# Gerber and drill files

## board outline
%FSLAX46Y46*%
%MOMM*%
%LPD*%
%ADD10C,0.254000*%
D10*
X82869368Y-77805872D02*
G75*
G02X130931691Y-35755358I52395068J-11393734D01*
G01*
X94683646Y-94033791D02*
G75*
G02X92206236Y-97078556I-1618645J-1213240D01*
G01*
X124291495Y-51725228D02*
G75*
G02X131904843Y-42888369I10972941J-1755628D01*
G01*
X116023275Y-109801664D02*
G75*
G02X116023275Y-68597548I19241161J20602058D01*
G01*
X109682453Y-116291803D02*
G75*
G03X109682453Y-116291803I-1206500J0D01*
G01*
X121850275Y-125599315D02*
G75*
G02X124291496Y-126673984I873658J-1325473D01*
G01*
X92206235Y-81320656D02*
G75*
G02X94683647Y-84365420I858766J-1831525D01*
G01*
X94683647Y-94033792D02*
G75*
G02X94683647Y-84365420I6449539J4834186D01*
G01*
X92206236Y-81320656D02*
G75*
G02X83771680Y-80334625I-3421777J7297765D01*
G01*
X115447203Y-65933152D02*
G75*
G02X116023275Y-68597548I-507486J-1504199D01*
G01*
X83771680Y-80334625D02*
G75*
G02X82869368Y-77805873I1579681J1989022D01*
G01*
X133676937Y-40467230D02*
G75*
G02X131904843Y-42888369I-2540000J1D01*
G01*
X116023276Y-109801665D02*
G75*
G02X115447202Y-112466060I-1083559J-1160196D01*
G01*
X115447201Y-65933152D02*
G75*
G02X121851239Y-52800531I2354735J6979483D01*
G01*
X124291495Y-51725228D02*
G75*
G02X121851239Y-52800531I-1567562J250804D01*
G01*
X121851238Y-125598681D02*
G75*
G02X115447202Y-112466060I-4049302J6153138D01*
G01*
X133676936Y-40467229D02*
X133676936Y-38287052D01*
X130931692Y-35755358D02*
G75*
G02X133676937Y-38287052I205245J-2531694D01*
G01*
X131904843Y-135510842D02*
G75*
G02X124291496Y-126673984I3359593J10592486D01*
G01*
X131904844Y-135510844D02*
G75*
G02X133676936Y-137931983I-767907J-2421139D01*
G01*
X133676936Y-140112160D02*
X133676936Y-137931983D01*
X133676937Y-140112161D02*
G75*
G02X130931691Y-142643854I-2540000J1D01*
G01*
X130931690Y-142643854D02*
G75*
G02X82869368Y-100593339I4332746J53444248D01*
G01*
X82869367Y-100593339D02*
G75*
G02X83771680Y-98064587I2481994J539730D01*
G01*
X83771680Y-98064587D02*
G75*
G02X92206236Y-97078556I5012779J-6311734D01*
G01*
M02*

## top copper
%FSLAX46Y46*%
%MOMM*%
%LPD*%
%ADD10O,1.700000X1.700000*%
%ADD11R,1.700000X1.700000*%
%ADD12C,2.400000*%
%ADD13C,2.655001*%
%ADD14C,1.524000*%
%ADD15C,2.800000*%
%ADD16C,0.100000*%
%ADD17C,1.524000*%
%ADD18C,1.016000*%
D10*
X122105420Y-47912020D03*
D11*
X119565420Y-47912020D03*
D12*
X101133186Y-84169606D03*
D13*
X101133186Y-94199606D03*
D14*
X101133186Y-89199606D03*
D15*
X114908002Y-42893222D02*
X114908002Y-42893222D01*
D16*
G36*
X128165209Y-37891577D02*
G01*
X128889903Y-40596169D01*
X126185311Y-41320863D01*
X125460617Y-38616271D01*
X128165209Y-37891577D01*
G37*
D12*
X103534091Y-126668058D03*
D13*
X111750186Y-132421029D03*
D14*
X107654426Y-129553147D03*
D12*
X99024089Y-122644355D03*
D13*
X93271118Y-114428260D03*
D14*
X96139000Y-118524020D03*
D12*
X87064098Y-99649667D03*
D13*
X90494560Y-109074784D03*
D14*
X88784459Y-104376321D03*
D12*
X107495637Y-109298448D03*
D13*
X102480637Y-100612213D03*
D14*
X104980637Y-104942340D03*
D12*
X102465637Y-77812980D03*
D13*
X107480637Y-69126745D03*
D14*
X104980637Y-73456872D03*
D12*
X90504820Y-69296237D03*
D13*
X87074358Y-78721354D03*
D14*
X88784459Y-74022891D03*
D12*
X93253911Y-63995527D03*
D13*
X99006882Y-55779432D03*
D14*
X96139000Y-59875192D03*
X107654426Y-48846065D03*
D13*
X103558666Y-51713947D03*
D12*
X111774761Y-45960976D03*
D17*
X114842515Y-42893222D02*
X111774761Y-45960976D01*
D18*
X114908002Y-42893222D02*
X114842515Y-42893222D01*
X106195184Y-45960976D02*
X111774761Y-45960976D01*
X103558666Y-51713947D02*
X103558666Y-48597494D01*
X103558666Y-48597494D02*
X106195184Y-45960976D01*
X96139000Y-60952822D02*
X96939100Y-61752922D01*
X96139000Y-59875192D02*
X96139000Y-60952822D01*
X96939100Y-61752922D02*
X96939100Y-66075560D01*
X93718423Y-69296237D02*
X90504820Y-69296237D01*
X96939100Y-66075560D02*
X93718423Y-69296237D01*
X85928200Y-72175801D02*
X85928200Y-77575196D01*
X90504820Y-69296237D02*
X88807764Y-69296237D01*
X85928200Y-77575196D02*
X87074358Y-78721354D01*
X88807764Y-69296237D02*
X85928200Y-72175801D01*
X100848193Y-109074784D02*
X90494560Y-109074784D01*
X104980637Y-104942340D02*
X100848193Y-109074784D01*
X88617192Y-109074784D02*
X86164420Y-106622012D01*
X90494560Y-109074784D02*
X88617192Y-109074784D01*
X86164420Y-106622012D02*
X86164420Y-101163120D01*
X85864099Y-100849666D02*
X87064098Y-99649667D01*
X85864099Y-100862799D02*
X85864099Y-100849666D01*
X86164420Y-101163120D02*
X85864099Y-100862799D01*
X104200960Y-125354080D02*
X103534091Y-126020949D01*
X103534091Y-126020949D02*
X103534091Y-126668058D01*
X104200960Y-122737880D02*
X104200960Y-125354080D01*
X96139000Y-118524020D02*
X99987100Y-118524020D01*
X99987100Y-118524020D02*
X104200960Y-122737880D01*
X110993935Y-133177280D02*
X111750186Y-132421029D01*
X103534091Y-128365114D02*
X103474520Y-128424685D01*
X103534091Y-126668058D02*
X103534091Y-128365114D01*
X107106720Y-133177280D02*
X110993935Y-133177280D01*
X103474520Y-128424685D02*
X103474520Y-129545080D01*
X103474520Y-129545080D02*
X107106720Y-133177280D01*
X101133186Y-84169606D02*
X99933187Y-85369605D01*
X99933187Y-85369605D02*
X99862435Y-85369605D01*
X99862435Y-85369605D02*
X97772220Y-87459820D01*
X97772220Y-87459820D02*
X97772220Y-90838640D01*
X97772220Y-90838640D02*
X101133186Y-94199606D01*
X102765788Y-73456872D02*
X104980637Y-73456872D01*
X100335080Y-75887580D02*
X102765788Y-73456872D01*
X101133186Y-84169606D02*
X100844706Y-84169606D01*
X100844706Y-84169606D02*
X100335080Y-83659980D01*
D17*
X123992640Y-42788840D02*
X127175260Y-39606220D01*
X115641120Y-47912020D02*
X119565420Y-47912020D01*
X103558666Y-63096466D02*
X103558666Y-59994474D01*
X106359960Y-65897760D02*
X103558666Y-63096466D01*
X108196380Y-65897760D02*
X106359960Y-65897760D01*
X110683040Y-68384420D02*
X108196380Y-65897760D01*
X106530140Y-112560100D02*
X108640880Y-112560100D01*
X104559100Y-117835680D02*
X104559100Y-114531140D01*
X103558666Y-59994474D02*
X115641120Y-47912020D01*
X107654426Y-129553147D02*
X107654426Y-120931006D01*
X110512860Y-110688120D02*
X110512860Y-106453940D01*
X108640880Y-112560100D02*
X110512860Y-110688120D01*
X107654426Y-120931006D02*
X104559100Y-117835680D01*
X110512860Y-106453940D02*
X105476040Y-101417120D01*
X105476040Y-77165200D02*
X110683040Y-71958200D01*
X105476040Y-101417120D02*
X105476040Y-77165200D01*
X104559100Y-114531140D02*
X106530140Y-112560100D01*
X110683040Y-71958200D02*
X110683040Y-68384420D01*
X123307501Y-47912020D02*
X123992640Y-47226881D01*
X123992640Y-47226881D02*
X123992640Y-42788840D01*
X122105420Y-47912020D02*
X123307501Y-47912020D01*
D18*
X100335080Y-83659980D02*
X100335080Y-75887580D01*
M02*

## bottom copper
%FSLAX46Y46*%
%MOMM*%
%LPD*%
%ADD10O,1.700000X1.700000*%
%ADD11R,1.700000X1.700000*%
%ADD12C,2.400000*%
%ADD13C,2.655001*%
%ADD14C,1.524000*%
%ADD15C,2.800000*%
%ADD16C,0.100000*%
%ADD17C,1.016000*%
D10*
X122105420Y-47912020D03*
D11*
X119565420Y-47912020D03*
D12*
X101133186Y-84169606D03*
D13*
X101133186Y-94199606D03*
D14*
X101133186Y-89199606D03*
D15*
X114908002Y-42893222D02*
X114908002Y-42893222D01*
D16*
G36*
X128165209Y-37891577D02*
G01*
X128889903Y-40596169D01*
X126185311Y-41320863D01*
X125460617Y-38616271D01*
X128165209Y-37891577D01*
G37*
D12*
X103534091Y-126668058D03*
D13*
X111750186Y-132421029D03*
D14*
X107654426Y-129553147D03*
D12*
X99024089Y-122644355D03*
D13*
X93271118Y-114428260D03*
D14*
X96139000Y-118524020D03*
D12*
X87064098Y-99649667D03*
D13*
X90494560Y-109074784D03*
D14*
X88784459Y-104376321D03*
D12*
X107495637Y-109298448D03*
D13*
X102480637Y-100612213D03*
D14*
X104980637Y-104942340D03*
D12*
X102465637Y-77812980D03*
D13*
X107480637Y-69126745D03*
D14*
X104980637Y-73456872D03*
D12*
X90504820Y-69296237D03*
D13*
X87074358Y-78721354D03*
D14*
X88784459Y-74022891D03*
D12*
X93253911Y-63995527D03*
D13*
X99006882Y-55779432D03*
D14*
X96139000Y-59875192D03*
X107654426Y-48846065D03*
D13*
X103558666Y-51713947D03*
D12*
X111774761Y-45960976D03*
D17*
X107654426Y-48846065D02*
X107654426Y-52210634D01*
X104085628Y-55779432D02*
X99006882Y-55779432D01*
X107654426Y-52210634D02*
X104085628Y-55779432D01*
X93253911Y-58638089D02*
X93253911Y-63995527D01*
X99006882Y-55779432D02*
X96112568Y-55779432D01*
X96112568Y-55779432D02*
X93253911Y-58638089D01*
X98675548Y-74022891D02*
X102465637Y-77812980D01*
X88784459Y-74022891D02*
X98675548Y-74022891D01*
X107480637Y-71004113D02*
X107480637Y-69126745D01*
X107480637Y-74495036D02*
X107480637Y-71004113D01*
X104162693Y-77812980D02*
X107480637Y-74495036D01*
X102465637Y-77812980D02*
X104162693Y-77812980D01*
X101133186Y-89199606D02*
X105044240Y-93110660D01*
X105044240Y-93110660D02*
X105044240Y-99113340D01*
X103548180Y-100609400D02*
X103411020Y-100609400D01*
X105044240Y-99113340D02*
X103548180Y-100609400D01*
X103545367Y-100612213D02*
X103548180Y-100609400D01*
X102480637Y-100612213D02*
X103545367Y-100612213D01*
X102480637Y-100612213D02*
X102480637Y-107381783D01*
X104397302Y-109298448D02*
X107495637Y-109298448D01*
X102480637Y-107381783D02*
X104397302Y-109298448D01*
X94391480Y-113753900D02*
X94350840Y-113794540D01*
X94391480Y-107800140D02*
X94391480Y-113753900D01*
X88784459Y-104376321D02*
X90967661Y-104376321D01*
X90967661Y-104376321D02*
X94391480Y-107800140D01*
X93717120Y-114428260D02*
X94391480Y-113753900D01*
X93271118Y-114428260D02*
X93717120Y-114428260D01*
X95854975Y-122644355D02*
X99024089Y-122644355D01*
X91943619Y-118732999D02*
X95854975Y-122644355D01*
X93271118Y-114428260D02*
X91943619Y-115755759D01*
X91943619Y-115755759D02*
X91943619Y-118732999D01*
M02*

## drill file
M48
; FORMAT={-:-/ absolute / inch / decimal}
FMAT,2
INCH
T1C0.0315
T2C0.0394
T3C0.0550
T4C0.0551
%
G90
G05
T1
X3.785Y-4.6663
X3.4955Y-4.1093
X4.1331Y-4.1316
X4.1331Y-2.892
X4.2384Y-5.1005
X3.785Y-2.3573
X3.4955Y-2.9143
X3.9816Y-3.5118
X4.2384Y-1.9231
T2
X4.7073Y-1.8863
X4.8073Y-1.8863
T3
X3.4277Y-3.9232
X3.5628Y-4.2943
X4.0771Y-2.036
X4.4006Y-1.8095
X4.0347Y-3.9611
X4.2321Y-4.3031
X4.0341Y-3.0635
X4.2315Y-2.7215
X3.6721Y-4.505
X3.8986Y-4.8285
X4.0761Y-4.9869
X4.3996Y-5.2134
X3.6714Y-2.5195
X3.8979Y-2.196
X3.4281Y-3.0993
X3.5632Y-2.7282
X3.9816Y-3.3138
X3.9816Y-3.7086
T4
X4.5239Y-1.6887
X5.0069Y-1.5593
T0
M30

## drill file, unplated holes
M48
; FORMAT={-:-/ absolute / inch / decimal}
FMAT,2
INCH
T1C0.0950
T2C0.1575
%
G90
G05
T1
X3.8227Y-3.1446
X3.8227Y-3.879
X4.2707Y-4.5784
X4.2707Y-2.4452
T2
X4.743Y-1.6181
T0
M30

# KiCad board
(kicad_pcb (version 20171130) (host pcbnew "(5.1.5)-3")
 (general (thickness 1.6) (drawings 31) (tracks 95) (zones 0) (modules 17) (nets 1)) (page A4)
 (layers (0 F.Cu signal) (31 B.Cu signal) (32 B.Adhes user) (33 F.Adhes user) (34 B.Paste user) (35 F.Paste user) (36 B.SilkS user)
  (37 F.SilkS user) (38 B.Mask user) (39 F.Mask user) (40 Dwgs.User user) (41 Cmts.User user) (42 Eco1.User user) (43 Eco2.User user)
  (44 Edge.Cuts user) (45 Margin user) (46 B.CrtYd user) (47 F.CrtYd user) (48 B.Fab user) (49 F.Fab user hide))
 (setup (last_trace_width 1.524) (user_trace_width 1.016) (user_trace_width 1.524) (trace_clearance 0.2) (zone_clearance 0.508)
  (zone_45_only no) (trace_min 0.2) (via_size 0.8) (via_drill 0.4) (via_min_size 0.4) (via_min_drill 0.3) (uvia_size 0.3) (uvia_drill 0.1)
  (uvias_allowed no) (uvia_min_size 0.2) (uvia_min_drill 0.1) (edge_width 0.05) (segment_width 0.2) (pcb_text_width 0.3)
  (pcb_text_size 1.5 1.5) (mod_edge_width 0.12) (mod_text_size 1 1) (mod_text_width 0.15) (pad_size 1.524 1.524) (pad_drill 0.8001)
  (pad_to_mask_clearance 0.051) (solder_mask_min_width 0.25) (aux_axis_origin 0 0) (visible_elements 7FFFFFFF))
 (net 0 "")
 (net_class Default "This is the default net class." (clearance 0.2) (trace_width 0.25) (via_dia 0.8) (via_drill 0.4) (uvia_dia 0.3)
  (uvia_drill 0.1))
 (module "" (layer F.Cu) (at 121.2342 50.3174)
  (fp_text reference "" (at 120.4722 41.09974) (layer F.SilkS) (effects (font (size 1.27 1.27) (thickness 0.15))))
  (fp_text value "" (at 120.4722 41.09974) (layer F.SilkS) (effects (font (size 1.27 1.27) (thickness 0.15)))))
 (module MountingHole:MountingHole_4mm (layer F.Cu) (at 120.4722 41.09974)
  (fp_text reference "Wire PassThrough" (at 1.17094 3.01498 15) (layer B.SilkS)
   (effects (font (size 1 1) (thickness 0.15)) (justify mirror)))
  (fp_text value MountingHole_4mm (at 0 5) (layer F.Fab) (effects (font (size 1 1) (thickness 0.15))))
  (pad "" np_thru_hole circle (at 0 0) (size 4 4) (drill 4) (layers *.Cu *.Mask)))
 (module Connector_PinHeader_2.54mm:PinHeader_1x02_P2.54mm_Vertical (layer F.Cu) (at 119.56542 47.91202 90)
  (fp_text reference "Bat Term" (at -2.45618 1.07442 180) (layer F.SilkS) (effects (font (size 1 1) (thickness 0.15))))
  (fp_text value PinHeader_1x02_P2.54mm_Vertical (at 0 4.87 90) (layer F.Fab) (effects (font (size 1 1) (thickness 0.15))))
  (pad 2 thru_hole oval (at 0 2.54 90) (size 1.7 1.7) (drill 1) (layers *.Cu *.Mask))
  (pad 1 thru_hole rect (at 0 0 90) (size 1.7 1.7) (drill 1) (layers *.Cu *.Mask)))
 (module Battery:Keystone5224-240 (layer F.Cu) (at 101.133186 89.199606)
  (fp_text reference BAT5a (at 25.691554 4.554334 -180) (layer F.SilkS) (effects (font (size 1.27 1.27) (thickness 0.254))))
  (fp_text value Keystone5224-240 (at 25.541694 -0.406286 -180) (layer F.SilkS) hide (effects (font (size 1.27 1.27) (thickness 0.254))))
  (pad 2 thru_hole circle (at 0 -5.03) (size 2.4 2.4) (drill 1.397) (layers *.Cu *.Mask))
  (pad 1 thru_hole circle (at 0 5) (size 2.655001 2.655001) (drill 1.397) (layers *.Cu *.Mask))
  (pad 3 thru_hole circle (at 0 0) (size 1.524 1.524) (drill 0.8001) (layers *.Cu *.Mask)))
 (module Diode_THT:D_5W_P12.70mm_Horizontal (layer F.Cu) (at 127.17526 39.60622 195)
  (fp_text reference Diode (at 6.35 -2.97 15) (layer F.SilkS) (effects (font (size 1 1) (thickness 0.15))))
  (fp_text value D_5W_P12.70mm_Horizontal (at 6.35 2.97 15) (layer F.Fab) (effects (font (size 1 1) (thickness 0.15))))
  (pad 2 thru_hole oval (at 12.7 0 195) (size 2.8 2.8) (drill 1.4) (layers *.Cu *.Mask))
  (pad 1 thru_hole rect (at 0 0 195) (size 2.8 2.8) (drill 1.4) (layers *.Cu *.Mask)))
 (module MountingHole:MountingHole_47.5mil (layer F.Cu) (at 108.475953 116.291803)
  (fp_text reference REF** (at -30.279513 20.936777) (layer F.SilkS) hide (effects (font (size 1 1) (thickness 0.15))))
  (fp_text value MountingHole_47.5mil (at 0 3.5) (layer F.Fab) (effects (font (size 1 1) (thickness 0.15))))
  (pad "" np_thru_hole circle (at 0 0) (size 2.413 2.413) (drill 2.413) (layers *.Cu *.Mask)))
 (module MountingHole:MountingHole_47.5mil (layer F.Cu) (at 97.096838 98.527587)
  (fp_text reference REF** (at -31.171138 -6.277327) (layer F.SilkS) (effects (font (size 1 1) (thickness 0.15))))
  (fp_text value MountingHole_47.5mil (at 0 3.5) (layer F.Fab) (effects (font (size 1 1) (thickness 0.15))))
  (pad "" np_thru_hole circle (at 0 0) (size 2.413 2.413) (drill 2.413) (layers *.Cu *.Mask)))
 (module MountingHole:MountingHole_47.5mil (layer F.Cu) (at 97.096838 79.871625)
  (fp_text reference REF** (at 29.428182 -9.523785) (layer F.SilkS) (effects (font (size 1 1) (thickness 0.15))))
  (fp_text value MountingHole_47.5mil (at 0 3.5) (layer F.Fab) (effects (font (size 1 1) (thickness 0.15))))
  (pad "" np_thru_hole circle (at 0 0) (size 2.413 2.413) (drill 2.413) (layers *.Cu *.Mask)))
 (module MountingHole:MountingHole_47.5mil (layer F.Cu) (at 108.475953 62.107409)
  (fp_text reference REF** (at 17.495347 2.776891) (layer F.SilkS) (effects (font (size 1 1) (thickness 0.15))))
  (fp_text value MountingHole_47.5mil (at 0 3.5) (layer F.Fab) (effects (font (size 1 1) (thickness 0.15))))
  (pad "" np_thru_hole circle (at 0 0) (size 2.413 2.413) (drill 2.413) (layers *.Cu *.Mask)))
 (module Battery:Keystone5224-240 (layer F.Cu) (at 107.654426 129.553147 55)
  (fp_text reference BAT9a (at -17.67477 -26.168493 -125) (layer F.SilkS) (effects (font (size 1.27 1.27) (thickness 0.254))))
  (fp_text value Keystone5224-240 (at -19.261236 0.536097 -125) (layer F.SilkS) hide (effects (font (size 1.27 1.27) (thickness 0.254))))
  (pad 2 thru_hole circle (at 0 -5.03 55) (size 2.4 2.4) (drill 1.397) (layers *.Cu *.Mask))
  (pad 1 thru_hole circle (at 0 5 55) (size 2.655001 2.655001) (drill 1.397) (layers *.Cu *.Mask))
  (pad 3 thru_hole circle (at 0 0 55) (size 1.524 1.524) (drill 0.8001) (layers *.Cu *.Mask)))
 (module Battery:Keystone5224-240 (layer B.Cu) (at 96.139 118.52402 35)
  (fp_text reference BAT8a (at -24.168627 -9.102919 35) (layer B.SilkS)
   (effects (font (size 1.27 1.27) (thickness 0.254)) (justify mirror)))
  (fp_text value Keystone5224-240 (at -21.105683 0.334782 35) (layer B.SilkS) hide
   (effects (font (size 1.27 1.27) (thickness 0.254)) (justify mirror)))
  (pad 2 thru_hole circle (at 0 5.03 35) (size 2.4 2.4) (drill 1.397) (layers *.Cu *.Mask))
  (pad 1 thru_hole circle (at 0 -5 35) (size 2.655001 2.655001) (drill 1.397) (layers *.Cu *.Mask))
  (pad 3 thru_hole circle (at 0 0 35) (size 1.524 1.524) (drill 0.8001) (layers *.Cu *.Mask)))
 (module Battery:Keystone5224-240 (layer F.Cu) (at 88.784459 104.376321 20)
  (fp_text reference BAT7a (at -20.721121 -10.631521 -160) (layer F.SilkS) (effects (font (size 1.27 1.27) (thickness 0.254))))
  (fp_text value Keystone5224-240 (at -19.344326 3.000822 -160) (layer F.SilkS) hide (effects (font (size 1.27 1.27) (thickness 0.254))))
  (pad 2 thru_hole circle (at 0 -5.03 20) (size 2.4 2.4) (drill 1.397) (layers *.Cu *.Mask))
  (pad 1 thru_hole circle (at 0 5 20) (size 2.655001 2.655001) (drill 1.397) (layers *.Cu *.Mask))
  (pad 3 thru_hole circle (at 0 0 20) (size 1.524 1.524) (drill 0.8001) (layers *.Cu *.Mask)))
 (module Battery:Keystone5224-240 (layer B.Cu) (at 104.980637 104.94234 30)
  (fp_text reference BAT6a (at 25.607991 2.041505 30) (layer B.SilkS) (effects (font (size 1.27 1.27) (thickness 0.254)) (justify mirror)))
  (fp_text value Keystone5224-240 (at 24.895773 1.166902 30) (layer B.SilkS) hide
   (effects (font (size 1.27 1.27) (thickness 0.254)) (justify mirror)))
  (pad 2 thru_hole circle (at 0 5.03 30) (size 2.4 2.4) (drill 1.397) (layers *.Cu *.Mask))
  (pad 1 thru_hole circle (at 0 -5 30) (size 2.655001 2.655001) (drill 1.397) (layers *.Cu *.Mask))
  (pad 3 thru_hole circle (at 0 0 30) (size 1.524 1.524) (drill 0.8001) (layers *.Cu *.Mask)))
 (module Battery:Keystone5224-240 (layer B.Cu) (at 104.980637 73.456872 330)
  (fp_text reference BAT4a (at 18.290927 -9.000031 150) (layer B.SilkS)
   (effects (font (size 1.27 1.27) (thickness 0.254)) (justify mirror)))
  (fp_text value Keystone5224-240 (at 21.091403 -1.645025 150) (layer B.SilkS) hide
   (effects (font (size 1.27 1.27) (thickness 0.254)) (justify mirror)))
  (pad 2 thru_hole circle (at 0 5.03 330) (size 2.4 2.4) (drill 1.397) (layers *.Cu *.Mask))
  (pad 1 thru_hole circle (at 0 -5 330) (size 2.655001 2.655001) (drill 1.397) (layers *.Cu *.Mask))
  (pad 3 thru_hole circle (at 0 0 330) (size 1.524 1.524) (drill 0.8001) (layers *.Cu *.Mask)))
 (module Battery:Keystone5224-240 (layer F.Cu) (at 88.784459 74.022891 340)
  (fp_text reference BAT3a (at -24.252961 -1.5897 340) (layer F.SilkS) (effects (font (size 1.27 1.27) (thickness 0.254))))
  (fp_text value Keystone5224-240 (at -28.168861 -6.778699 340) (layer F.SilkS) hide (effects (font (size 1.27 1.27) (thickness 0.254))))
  (pad 2 thru_hole circle (at 0 -5.03 340) (size 2.4 2.4) (drill 1.397) (layers *.Cu *.Mask))
  (pad 1 thru_hole circle (at 0 5 340) (size 2.655001 2.655001) (drill 1.397) (layers *.Cu *.Mask))
  (pad 3 thru_hole circle (at 0 0 340) (size 1.524 1.524) (drill 0.8001) (layers *.Cu *.Mask)))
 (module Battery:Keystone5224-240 (layer B.Cu) (at 96.139 59.875192 325)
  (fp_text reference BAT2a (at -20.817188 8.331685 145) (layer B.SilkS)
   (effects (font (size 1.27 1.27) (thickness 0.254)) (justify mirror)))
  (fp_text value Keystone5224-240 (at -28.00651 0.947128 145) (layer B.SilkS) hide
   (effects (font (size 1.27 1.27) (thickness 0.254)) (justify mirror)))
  (pad 2 thru_hole circle (at 0 5.03 325) (size 2.4 2.4) (drill 1.397) (layers *.Cu *.Mask))
  (pad 1 thru_hole circle (at 0 -5 325) (size 2.655001 2.655001) (drill 1.397) (layers *.Cu *.Mask))
  (pad 3 thru_hole circle (at 0 0 325) (size 1.524 1.524) (drill 0.8001) (layers *.Cu *.Mask)))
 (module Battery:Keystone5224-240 (layer F.Cu) (at 107.654426 48.846065 305)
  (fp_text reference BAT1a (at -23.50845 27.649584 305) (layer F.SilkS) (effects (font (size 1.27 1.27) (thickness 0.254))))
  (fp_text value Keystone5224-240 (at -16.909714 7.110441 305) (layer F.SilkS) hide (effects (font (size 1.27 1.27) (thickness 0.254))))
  (pad 3 thru_hole circle (at 0 0 305) (size 1.524 1.524) (drill 0.8001) (layers *.Cu *.Mask))
  (pad 1 thru_hole circle (at 0 5 305) (size 2.655001 2.655001) (drill 1.397) (layers *.Cu *.Mask))
  (pad 2 thru_hole circle (at 0 -5.03 305) (size 2.4 2.4) (drill 1.397) (layers *.Cu *.Mask)))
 (gr_arc (start 135.264436 89.199606) (end 130.931691 35.755358) (angle -73.09671633) (layer Edge.Cuts) (width 0.254))
 (gr_arc (start 93.065001 95.247031) (end 92.206236 97.078556) (angle -151.9739674) (layer Edge.Cuts) (width 0.254))
 (gr_arc (start 135.264436 53.480856) (end 131.904843 42.888369) (angle -63.31259973) (layer Edge.Cuts) (width 0.254))
 (gr_arc (start 135.264436 89.199606) (end 116.023275 68.597548) (angle -93.91250265) (layer Edge.Cuts) (width 0.254))
 (gr_circle (center 108.475953 116.291803) (end 109.682453 116.291803) (layer Edge.Cuts) (width 0.254))
 (gr_arc (start 122.723933 126.924788) (end 124.291496 126.673984) (angle -114.3) (layer Edge.Cuts) (width 0.254))
 (gr_arc (start 93.065001 83.152181) (end 94.683647 84.36542) (angle -151.9739674) (layer Edge.Cuts) (width 0.254))
 (gr_arc (start 101.133186 89.199606) (end 94.683647 84.36542) (angle -73.70603612) (layer Edge.Cuts) (width 0.254))
 (gr_arc (start 88.784459 74.022891) (end 83.77168 80.334625) (angle -63.5775508) (layer Edge.Cuts) (width 0.254))
 (gr_arc (start 114.939717 67.437351) (end 116.023275 68.597548) (angle -118.3129136) (layer Edge.Cuts) (width 0.254))
 (gr_arc (start 85.351361 78.345603) (end 82.869368 77.805873) (angle -63.8118281) (layer Edge.Cuts) (width 0.254))
 (gr_arc (start 131.136937 40.467229) (end 131.904843 42.888369) (angle -72.40266339) (layer Edge.Cuts) (width 0.254))
 (gr_arc (start 114.939717 110.961861) (end 115.447202 112.46606) (angle -118.3129136) (layer Edge.Cuts) (width 0.254))
 (gr_arc (start 117.801936 58.953669) (end 121.851239 52.800531) (angle -194.7050695) (layer Edge.Cuts) (width 0.254))
 (gr_arc (start 122.723933 51.474424) (end 121.851239 52.800531) (angle -114.2583435) (layer Edge.Cuts) (width 0.254))
 (gr_arc (start 117.801936 119.445543) (end 115.447202 112.46606) (angle -194.7050695) (layer Edge.Cuts) (width 0.254))
 (gr_line (start 133.676936 40.467229) (end 133.676936 38.287052) (layer Edge.Cuts) (width 0.254))
 (gr_arc (start 131.136937 38.287052) (end 133.676937 38.287052) (angle -94.63485415) (layer Edge.Cuts) (width 0.254))
 (gr_arc (start 135.264436 124.918356) (end 124.291496 126.673984) (angle -63.31259973) (layer Edge.Cuts) (width 0.254))
 (gr_arc (start 131.136937 137.931983) (end 133.676936 137.931983) (angle -72.40266339) (layer Edge.Cuts) (width 0.254))
 (gr_line (start 133.676936 140.11216) (end 133.676936 137.931983) (layer Edge.Cuts) (width 0.254))
 (gr_arc (start 131.136937 140.11216) (end 130.931691 142.643854) (angle -94.63485415) (layer Edge.Cuts) (width 0.254))
 (gr_arc (start 135.264436 89.199606) (end 82.869368 100.593339) (angle -73.09671633) (layer Edge.Cuts) (width 0.254))
 (gr_arc (start 85.351361 100.053609) (end 83.77168 98.064587) (angle -63.8118281) (layer Edge.Cuts) (width 0.254))
 (gr_arc (start 88.784459 104.376321) (end 92.206236 97.078556) (angle -63.5775508) (layer Edge.Cuts) (width 0.254))
 (segment (start 114.842515 42.893222) (end 111.774761 45.960976) (width 1.524) (layer F.Cu) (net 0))
 (segment (start 114.908002 42.893222) (end 114.842515 42.893222) (width 1.016) (layer F.Cu) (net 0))
 (segment (start 106.195184 45.960976) (end 111.774761 45.960976) (width 1.016) (layer F.Cu) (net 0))
 (segment (start 103.558666 51.713947) (end 103.558666 48.597494) (width 1.016) (layer F.Cu) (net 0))
 (segment (start 103.558666 48.597494) (end 106.195184 45.960976) (width 1.016) (layer F.Cu) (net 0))
 (segment (start 107.654426 48.846065) (end 107.654426 52.210634) (width 1.016) (layer B.Cu) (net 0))
 (segment (start 104.085628 55.779432) (end 99.006882 55.779432) (width 1.016) (layer B.Cu) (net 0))
 (segment (start 107.654426 52.210634) (end 104.085628 55.779432) (width 1.016) (layer B.Cu) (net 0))
 (segment (start 93.253911 58.638089) (end 93.253911 63.995527) (width 1.016) (layer B.Cu) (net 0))
 (segment (start 99.006882 55.779432) (end 96.112568 55.779432) (width 1.016) (layer B.Cu) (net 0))
 (segment (start 96.112568 55.779432) (end 93.253911 58.638089) (width 1.016) (layer B.Cu) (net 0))
 (segment (start 96.139 60.952822) (end 96.9391 61.752922) (width 1.016) (layer F.Cu) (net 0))
 (segment (start 96.139 59.875192) (end 96.139 60.952822) (width 1.016) (layer F.Cu) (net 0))
 (segment (start 96.9391 61.752922) (end 96.9391 66.07556) (width 1.016) (layer F.Cu) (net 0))
 (segment (start 93.718423 69.296237) (end 90.50482 69.296237) (width 1.016) (layer F.Cu) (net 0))
 (segment (start 96.9391 66.07556) (end 93.718423 69.296237) (width 1.016) (layer F.Cu) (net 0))
 (segment (start 85.9282 72.175801) (end 85.9282 77.575196) (width 1.016) (layer F.Cu) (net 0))
 (segment (start 90.50482 69.296237) (end 88.807764 69.296237) (width 1.016) (layer F.Cu) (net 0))
 (segment (start 85.9282 77.575196) (end 87.074358 78.721354) (width 1.016) (layer F.Cu) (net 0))
 (segment (start 88.807764 69.296237) (end 85.9282 72.175801) (width 1.016) (layer F.Cu) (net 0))
 (segment (start 100.848193 109.074784) (end 90.49456 109.074784) (width 1.016) (layer F.Cu) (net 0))
 (segment (start 104.980637 104.94234) (end 100.848193 109.074784) (width 1.016) (layer F.Cu) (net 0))
 (segment (start 88.617192 109.074784) (end 86.16442 106.622012) (width 1.016) (layer F.Cu) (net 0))
 (segment (start 90.49456 109.074784) (end 88.617192 109.074784) (width 1.016) (layer F.Cu) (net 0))
 (segment (start 86.16442 106.622012) (end 86.16442 101.16312) (width 1.016) (layer F.Cu) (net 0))
 (segment (start 85.864099 100.849666) (end 87.064098 99.649667) (width 1.016) (layer F.Cu) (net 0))
 (segment (start 85.864099 100.862799) (end 85.864099 100.849666) (width 1.016) (layer F.Cu) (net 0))
 (segment (start 86.16442 101.16312) (end 85.864099 100.862799) (width 1.016) (layer F.Cu) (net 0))
 (segment (start 104.20096 125.35408) (end 103.534091 126.020949) (width 1.016) (layer F.Cu) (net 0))
 (segment (start 103.534091 126.020949) (end 103.534091 126.668058) (width 1.016) (layer F.Cu) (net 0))
 (segment (start 104.20096 122.73788) (end 104.20096 125.35408) (width 1.016) (layer F.Cu) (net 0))
 (segment (start 96.139 118.52402) (end 99.9871 118.52402) (width 1.016) (layer F.Cu) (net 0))
 (segment (start 99.9871 118.52402) (end 104.20096 122.73788) (width 1.016) (layer F.Cu) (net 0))
 (segment (start 110.993935 133.17728) (end 111.750186 132.421029) (width 1.016) (layer F.Cu) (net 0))
 (segment (start 103.534091 128.365114) (end 103.47452 128.424685) (width 1.016) (layer F.Cu) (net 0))
 (segment (start 103.534091 126.668058) (end 103.534091 128.365114) (width 1.016) (layer F.Cu) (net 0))
 (segment (start 107.10672 133.17728) (end 110.993935 133.17728) (width 1.016) (layer F.Cu) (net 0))
 (segment (start 103.47452 128.424685) (end 103.47452 129.54508) (width 1.016) (layer F.Cu) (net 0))
 (segment (start 103.47452 129.54508) (end 107.10672 133.17728) (width 1.016) (layer F.Cu) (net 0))
 (segment (start 98.675548 74.022891) (end 102.465637 77.81298) (width 1.016) (layer B.Cu) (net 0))
 (segment (start 88.784459 74.022891) (end 98.675548 74.022891) (width 1.016) (layer B.Cu) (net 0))
 (segment (start 107.480637 71.004113) (end 107.480637 69.126745) (width 1.016) (layer B.Cu) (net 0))
 (segment (start 107.480637 74.495036) (end 107.480637 71.004113) (width 1.016) (layer B.Cu) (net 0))
 (segment (start 104.162693 77.81298) (end 107.480637 74.495036) (width 1.016) (layer B.Cu) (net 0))
 (segment (start 102.465637 77.81298) (end 104.162693 77.81298) (width 1.016) (layer B.Cu) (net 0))
 (segment (start 101.133186 89.199606) (end 105.04424 93.11066) (width 1.016) (layer B.Cu) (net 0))
 (segment (start 105.04424 93.11066) (end 105.04424 99.11334) (width 1.016) (layer B.Cu) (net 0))
 (segment (start 103.54818 100.6094) (end 103.41102 100.6094) (width 1.016) (layer B.Cu) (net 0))
 (segment (start 105.04424 99.11334) (end 103.54818 100.6094) (width 1.016) (layer B.Cu) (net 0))
 (segment (start 103.545367 100.612213) (end 103.54818 100.6094) (width 1.016) (layer B.Cu) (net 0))
 (segment (start 102.480637 100.612213) (end 103.545367 100.612213) (width 1.016) (layer B.Cu) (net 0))
 (segment (start 102.480637 100.612213) (end 102.480637 107.381783) (width 1.016) (layer B.Cu) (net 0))
 (segment (start 104.397302 109.298448) (end 107.495637 109.298448) (width 1.016) (layer B.Cu) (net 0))
 (segment (start 102.480637 107.381783) (end 104.397302 109.298448) (width 1.016) (layer B.Cu) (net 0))
 (segment (start 94.39148 113.7539) (end 94.35084 113.79454) (width 1.016) (layer B.Cu) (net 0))
 (segment (start 94.39148 107.80014) (end 94.39148 113.7539) (width 1.016) (layer B.Cu) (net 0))
 (segment (start 88.784459 104.376321) (end 90.967661 104.376321) (width 1.016) (layer B.Cu) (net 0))
 (segment (start 90.967661 104.376321) (end 94.39148 107.80014) (width 1.016) (layer B.Cu) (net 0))
 (segment (start 93.71712 114.42826) (end 94.39148 113.7539) (width 1.016) (layer B.Cu) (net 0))
 (segment (start 93.271118 114.42826) (end 93.71712 114.42826) (width 1.016) (layer B.Cu) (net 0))
 (segment (start 95.854975 122.644355) (end 99.024089 122.644355) (width 1.016) (layer B.Cu) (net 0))
 (segment (start 91.943619 118.732999) (end 95.854975 122.644355) (width 1.016) (layer B.Cu) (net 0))
 (segment (start 93.271118 114.42826) (end 91.943619 115.755759) (width 1.016) (layer B.Cu) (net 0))
 (segment (start 91.943619 115.755759) (end 91.943619 118.732999) (width 1.016) (layer B.Cu) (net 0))
 (segment (start 101.133186 84.169606) (end 99.933187 85.369605) (width 1.016) (layer F.Cu) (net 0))
 (segment (start 99.933187 85.369605) (end 99.862435 85.369605) (width 1.016) (layer F.Cu) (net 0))
 (segment (start 99.862435 85.369605) (end 97.77222 87.45982) (width 1.016) (layer F.Cu) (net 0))
 (segment (start 97.77222 87.45982) (end 97.77222 90.83864) (width 1.016) (layer F.Cu) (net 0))
 (segment (start 97.77222 90.83864) (end 101.133186 94.199606) (width 1.016) (layer F.Cu) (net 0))
 (segment (start 102.765788 73.456872) (end 104.980637 73.456872) (width 1.016) (layer F.Cu) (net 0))
 (segment (start 100.33508 75.88758) (end 102.765788 73.456872) (width 1.016) (layer F.Cu) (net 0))
 (segment (start 101.133186 84.169606) (end 100.844706 84.169606) (width 1.016) (layer F.Cu) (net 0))
 (segment (start 100.844706 84.169606) (end 100.33508 83.65998) (width 1.016) (layer F.Cu) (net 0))
 (segment (start 123.99264 42.78884) (end 127.17526 39.60622) (width 1.524) (layer F.Cu) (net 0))
 (segment (start 115.64112 47.91202) (end 119.56542 47.91202) (width 1.524) (layer F.Cu) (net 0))
 (segment (start 103.558666 63.096466) (end 103.558666 59.994474) (width 1.524) (layer F.Cu) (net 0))
 (segment (start 106.35996 65.89776) (end 103.558666 63.096466) (width 1.524) (layer F.Cu) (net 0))
 (segment (start 108.19638 65.89776) (end 106.35996 65.89776) (width 1.524) (layer F.Cu) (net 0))
 (segment (start 110.68304 68.38442) (end 108.19638 65.89776) (width 1.524) (layer F.Cu) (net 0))
 (segment (start 106.53014 112.5601) (end 108.64088 112.5601) (width 1.524) (layer F.Cu) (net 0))
 (segment (start 104.5591 117.83568) (end 104.5591 114.53114) (width 1.524) (layer F.Cu) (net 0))
 (segment (start 103.558666 59.994474) (end 115.64112 47.91202) (width 1.524) (layer F.Cu) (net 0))
 (segment (start 107.654426 129.553147) (end 107.654426 120.931006) (width 1.524) (layer F.Cu) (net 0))
 (segment (start 110.51286 110.68812) (end 110.51286 106.45394) (width 1.524) (layer F.Cu) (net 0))
 (segment (start 108.64088 112.5601) (end 110.51286 110.68812) (width 1.524) (layer F.Cu) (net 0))
 (segment (start 107.654426 120.931006) (end 104.5591 117.83568) (width 1.524) (layer F.Cu) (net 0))
 (segment (start 110.51286 106.45394) (end 105.47604 101.41712) (width 1.524) (layer F.Cu) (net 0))
 (segment (start 105.47604 77.1652) (end 110.68304 71.9582) (width 1.524) (layer F.Cu) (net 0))
 (segment (start 105.47604 101.41712) (end 105.47604 77.1652) (width 1.524) (layer F.Cu) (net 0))
 (segment (start 104.5591 114.53114) (end 106.53014 112.5601) (width 1.524) (layer F.Cu) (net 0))
 (segment (start 110.68304 71.9582) (end 110.68304 68.38442) (width 1.524) (layer F.Cu) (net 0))
 (segment (start 123.307501 47.91202) (end 123.99264 47.226881) (width 1.524) (layer F.Cu) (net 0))
 (segment (start 123.99264 47.226881) (end 123.99264 42.78884) (width 1.524) (layer F.Cu) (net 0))
 (segment (start 122.10542 47.91202) (end 123.307501 47.91202) (width 1.524) (layer F.Cu) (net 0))
 (segment (start 100.33508 83.65998) (end 100.33508 75.88758) (width 1.016) (layer F.Cu) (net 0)))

